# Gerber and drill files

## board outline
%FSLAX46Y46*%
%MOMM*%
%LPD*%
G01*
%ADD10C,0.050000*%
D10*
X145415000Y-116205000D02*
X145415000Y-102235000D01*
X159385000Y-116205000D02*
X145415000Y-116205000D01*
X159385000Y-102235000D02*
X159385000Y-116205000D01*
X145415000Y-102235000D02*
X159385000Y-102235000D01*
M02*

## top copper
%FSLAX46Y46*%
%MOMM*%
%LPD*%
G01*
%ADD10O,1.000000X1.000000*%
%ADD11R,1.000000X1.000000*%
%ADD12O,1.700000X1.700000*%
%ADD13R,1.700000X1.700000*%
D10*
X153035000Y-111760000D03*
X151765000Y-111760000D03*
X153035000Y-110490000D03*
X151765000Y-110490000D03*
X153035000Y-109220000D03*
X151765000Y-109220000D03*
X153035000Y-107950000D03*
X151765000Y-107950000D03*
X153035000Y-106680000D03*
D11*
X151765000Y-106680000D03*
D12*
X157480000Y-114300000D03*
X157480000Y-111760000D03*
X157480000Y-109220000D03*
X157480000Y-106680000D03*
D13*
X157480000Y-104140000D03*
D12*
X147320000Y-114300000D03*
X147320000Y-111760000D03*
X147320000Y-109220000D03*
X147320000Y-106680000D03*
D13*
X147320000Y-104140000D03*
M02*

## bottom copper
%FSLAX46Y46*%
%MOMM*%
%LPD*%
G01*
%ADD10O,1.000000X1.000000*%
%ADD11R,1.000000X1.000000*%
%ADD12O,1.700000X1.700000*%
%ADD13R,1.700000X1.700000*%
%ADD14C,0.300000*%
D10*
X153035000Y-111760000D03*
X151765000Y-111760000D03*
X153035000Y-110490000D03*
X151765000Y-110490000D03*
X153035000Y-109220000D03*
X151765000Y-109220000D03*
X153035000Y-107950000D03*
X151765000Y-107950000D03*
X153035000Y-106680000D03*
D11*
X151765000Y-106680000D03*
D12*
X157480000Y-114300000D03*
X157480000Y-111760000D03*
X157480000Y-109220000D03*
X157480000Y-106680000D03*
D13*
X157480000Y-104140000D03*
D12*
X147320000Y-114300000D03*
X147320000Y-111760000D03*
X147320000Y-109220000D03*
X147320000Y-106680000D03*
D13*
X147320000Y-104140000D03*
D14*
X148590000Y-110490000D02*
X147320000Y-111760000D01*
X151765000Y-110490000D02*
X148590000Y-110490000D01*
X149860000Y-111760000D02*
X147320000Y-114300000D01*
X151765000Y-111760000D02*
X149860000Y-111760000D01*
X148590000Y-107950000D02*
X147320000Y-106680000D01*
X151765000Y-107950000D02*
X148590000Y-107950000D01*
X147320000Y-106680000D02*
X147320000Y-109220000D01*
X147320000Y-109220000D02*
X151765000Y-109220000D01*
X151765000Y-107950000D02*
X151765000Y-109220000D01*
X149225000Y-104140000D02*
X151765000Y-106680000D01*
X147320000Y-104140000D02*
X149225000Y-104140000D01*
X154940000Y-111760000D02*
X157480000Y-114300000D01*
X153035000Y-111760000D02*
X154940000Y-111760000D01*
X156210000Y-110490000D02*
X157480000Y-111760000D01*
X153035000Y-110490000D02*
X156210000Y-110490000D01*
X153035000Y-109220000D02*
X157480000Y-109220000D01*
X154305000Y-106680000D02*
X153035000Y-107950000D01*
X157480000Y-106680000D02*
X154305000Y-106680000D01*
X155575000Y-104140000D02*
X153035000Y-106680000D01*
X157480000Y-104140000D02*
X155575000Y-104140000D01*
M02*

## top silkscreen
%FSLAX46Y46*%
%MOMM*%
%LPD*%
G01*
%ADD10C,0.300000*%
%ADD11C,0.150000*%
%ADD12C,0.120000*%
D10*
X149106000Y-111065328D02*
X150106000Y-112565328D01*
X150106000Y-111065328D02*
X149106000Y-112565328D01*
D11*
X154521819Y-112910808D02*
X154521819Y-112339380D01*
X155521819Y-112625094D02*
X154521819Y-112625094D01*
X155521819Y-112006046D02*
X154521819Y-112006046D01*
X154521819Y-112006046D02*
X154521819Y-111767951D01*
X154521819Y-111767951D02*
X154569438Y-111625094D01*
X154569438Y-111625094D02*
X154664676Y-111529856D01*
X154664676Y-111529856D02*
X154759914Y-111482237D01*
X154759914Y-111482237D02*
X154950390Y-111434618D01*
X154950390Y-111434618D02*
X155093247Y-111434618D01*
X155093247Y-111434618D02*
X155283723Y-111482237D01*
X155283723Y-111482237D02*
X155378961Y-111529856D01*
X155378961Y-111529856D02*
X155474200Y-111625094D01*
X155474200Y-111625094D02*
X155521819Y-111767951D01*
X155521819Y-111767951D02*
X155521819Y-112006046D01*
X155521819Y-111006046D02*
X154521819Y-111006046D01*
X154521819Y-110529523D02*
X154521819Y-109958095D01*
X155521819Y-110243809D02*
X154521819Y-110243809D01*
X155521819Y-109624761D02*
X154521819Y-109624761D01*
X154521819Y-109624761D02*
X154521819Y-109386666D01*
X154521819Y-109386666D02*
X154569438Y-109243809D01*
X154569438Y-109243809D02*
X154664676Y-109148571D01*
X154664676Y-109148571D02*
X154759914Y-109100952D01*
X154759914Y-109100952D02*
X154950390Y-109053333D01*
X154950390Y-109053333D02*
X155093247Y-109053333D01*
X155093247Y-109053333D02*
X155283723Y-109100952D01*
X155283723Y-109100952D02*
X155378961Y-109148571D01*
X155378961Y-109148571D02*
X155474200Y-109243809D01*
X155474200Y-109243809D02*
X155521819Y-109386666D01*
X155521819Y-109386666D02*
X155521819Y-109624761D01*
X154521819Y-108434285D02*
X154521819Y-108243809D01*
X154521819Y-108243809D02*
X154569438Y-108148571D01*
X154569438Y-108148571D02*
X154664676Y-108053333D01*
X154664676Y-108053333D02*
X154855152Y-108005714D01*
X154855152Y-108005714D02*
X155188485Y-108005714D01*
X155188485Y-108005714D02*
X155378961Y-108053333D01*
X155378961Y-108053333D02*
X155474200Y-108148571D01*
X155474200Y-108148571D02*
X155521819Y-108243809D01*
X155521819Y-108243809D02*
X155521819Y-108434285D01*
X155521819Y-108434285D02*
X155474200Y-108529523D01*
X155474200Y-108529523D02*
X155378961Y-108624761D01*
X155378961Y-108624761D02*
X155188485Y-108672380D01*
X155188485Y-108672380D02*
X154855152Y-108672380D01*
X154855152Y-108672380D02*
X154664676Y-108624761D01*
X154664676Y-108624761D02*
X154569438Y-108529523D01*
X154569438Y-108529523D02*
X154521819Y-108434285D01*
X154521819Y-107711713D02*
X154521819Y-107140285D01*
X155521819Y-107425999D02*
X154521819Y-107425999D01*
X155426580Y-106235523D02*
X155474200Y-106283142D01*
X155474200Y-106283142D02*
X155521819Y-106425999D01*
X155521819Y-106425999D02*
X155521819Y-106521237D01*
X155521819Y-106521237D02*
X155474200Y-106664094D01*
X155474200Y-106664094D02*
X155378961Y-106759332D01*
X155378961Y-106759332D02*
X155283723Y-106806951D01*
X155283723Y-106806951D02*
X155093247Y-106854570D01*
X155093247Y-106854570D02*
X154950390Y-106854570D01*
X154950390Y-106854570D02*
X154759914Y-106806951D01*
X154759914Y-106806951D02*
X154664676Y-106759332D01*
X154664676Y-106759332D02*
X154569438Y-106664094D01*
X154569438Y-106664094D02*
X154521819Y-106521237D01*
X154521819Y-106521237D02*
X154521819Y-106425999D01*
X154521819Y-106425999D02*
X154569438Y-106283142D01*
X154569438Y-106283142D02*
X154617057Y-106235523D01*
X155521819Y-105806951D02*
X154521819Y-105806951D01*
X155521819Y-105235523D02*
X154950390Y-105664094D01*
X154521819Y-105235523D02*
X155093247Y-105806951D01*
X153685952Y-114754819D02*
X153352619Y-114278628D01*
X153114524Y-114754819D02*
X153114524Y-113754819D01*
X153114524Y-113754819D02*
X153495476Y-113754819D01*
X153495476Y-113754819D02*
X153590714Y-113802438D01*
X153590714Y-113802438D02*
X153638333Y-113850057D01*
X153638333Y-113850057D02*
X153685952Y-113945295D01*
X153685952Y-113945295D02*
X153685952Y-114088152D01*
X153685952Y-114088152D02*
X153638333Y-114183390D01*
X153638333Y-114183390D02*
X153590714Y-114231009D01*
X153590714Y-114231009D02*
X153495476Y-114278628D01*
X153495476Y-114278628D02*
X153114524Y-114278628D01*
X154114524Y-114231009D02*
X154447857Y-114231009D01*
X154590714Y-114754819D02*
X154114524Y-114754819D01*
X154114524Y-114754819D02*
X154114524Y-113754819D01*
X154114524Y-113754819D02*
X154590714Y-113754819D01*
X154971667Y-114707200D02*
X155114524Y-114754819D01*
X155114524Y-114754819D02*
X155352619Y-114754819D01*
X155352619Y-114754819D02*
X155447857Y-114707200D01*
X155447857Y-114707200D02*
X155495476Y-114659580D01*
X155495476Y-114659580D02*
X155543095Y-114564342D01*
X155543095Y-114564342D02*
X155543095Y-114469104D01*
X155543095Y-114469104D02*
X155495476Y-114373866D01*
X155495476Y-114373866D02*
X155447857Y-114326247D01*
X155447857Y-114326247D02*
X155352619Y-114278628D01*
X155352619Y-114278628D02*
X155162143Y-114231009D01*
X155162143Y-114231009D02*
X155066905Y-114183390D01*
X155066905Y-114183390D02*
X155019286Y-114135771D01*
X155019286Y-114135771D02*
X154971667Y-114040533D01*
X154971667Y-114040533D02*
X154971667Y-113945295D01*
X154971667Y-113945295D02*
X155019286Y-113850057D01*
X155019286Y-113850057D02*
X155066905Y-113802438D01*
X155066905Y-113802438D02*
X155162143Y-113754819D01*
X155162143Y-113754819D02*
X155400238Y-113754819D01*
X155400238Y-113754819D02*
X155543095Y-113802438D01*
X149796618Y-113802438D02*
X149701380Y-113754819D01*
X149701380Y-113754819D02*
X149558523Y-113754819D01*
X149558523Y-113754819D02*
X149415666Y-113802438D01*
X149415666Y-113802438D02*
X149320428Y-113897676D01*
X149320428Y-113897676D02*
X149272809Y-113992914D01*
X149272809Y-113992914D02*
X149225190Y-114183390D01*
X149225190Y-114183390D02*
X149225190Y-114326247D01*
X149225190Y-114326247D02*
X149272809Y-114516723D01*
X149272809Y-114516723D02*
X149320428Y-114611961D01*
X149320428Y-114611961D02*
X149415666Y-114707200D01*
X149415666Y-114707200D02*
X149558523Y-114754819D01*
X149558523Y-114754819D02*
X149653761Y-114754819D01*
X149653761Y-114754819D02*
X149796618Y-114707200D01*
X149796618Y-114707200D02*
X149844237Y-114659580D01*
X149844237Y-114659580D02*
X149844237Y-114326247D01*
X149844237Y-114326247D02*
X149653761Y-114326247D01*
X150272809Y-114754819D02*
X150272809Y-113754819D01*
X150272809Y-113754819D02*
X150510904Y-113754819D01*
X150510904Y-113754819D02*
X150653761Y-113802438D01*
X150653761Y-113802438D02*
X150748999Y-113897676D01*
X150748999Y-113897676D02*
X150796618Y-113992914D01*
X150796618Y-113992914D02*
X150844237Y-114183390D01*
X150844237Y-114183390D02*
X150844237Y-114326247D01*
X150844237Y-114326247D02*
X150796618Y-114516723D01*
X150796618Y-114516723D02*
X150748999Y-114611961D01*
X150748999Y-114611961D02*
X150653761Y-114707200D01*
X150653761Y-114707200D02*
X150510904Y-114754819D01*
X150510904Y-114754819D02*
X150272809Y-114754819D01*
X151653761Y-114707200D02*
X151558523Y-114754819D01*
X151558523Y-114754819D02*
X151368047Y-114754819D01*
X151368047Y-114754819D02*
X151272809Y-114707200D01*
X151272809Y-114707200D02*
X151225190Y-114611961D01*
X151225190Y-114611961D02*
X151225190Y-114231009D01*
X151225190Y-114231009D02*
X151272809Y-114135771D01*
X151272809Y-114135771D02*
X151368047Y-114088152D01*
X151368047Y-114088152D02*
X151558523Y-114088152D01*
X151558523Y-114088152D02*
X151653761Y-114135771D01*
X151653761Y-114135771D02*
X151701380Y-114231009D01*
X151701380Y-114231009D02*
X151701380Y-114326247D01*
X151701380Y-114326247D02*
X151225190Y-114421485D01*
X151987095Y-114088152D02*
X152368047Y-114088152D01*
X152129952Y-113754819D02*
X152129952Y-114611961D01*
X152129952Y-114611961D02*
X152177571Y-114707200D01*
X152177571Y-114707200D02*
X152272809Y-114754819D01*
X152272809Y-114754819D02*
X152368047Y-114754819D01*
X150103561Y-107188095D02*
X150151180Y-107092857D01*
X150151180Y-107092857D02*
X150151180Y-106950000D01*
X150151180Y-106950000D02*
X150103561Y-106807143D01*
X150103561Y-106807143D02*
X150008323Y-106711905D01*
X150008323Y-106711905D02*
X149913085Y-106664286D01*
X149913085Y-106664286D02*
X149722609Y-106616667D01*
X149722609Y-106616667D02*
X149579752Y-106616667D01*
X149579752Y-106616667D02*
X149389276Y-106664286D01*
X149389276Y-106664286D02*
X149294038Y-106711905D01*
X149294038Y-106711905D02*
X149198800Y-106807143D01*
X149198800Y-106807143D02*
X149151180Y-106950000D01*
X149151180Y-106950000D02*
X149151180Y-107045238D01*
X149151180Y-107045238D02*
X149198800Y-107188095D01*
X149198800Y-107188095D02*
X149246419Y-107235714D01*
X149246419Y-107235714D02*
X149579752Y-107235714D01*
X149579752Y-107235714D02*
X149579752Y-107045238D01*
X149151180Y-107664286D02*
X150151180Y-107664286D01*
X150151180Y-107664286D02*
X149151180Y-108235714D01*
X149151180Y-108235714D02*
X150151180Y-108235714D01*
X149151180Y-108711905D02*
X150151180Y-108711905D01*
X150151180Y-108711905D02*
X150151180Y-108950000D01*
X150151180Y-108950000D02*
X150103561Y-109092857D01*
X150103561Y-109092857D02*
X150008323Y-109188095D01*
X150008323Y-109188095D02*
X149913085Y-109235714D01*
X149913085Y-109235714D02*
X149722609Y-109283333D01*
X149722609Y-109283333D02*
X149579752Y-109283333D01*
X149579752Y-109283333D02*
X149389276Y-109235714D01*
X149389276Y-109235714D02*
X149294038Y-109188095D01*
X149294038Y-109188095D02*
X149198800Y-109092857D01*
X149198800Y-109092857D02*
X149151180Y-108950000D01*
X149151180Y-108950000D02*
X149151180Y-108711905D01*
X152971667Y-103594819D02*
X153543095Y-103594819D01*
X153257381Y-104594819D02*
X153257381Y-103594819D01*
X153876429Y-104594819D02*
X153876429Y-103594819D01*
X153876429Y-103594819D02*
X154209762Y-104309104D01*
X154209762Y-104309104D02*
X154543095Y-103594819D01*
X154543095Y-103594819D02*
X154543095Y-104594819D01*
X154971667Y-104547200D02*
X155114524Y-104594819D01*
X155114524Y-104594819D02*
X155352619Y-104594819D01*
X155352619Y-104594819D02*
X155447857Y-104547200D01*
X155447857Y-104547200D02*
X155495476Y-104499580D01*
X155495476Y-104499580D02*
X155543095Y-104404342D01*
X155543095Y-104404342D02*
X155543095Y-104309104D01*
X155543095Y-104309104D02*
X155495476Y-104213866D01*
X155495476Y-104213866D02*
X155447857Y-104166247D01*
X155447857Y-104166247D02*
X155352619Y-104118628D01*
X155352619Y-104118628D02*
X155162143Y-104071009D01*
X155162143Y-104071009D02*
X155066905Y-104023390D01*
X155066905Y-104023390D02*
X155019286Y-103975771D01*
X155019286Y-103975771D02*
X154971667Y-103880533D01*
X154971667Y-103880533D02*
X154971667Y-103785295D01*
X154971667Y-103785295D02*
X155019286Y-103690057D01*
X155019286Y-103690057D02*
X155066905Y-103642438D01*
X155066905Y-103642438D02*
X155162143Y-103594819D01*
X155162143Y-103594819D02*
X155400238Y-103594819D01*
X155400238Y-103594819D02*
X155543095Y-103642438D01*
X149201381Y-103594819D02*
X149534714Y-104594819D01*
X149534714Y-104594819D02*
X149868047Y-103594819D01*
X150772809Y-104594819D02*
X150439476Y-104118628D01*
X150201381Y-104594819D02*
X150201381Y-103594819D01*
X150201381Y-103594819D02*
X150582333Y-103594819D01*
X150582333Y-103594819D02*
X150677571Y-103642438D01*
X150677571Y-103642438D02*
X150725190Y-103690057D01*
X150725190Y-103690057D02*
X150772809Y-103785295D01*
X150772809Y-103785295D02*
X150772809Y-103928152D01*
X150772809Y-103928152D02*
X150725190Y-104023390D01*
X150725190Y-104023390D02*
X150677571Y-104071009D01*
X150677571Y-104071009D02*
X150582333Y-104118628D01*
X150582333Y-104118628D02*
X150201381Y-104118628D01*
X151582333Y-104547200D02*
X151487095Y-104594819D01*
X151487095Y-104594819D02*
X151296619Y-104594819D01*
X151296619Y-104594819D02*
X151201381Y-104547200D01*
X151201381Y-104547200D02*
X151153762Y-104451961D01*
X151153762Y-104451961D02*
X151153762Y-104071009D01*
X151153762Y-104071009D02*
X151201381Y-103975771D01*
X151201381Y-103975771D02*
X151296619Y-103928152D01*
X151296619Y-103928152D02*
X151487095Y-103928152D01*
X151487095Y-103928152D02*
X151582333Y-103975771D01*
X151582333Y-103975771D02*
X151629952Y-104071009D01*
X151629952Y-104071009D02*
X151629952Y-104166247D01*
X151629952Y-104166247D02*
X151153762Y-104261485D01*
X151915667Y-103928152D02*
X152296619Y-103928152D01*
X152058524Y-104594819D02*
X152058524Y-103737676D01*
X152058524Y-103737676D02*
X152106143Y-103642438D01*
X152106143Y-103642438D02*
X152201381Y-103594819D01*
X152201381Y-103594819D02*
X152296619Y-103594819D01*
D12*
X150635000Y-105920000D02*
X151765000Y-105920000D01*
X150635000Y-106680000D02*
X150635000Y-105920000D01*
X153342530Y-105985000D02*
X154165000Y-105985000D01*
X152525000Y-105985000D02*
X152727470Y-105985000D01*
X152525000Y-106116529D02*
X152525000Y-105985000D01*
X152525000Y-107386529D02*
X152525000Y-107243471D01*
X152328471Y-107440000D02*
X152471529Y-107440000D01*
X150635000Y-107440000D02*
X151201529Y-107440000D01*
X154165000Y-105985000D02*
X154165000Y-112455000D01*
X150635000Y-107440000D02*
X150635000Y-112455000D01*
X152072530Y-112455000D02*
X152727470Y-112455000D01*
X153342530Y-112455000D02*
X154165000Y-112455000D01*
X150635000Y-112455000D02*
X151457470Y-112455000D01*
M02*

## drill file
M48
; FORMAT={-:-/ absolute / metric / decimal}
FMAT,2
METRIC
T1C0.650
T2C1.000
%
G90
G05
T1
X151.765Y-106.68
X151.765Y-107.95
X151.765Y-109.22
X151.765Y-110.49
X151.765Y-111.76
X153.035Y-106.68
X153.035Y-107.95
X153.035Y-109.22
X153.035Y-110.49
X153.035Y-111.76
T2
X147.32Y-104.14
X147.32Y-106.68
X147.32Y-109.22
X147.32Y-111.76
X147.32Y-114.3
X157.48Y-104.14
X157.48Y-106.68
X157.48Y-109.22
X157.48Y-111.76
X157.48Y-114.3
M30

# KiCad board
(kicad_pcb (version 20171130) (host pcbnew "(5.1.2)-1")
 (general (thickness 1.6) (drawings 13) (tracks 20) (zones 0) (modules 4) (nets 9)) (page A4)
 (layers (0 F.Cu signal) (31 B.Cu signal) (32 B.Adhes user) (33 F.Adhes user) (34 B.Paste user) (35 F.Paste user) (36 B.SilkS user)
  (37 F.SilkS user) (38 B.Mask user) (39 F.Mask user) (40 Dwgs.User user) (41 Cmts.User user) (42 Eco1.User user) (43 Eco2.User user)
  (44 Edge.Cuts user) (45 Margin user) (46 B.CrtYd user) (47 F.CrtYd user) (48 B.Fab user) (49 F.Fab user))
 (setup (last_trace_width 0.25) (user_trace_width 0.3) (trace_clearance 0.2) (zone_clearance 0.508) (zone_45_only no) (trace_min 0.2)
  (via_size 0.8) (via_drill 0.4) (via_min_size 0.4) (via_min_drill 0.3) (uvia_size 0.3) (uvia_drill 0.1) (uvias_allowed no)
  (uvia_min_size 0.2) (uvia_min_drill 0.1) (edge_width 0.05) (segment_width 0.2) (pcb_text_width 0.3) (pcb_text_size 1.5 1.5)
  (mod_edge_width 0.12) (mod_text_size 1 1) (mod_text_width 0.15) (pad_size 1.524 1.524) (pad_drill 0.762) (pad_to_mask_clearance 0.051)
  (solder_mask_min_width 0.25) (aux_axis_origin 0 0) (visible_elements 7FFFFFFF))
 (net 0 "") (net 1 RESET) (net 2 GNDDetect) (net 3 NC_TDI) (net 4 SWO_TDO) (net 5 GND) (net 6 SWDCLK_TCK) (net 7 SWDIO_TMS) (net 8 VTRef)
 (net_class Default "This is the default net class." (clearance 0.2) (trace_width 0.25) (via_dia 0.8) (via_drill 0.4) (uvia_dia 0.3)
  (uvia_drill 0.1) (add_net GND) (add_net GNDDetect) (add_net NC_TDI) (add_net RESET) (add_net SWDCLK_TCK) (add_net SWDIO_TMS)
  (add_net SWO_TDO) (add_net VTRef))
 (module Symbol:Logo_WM (layer B.Cu) (at 152.527 114.427)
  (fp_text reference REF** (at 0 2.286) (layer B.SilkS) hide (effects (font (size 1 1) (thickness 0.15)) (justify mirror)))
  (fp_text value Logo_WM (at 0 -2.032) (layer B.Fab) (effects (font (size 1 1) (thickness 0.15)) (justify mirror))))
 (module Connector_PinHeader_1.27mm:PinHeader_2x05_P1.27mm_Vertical (layer F.Cu) (at 151.765 106.68)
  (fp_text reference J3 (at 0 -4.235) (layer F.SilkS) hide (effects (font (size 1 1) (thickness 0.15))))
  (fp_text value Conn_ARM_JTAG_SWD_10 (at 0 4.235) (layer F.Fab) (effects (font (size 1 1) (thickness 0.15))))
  (fp_line (start -1.13 -0.76) (end 0 -0.76) (layer F.SilkS) (width 0.12))
  (fp_line (start -1.13 0) (end -1.13 -0.76) (layer F.SilkS) (width 0.12))
  (fp_line (start 1.57753 -0.695) (end 2.4 -0.695) (layer F.SilkS) (width 0.12))
  (fp_line (start 0.76 -0.695) (end 0.96247 -0.695) (layer F.SilkS) (width 0.12))
  (fp_line (start 0.76 -0.563471) (end 0.76 -0.695) (layer F.SilkS) (width 0.12))
  (fp_line (start 0.76 0.706529) (end 0.76 0.563471) (layer F.SilkS) (width 0.12))
  (fp_line (start 0.563471 0.76) (end 0.706529 0.76) (layer F.SilkS) (width 0.12))
  (fp_line (start -1.13 0.76) (end -0.563471 0.76) (layer F.SilkS) (width 0.12))
  (fp_line (start 2.4 -0.695) (end 2.4 5.775) (layer F.SilkS) (width 0.12))
  (fp_line (start -1.13 0.76) (end -1.13 5.775) (layer F.SilkS) (width 0.12))
  (fp_line (start 0.30753 5.775) (end 0.96247 5.775) (layer F.SilkS) (width 0.12))
  (fp_line (start 1.57753 5.775) (end 2.4 5.775) (layer F.SilkS) (width 0.12))
  (fp_line (start -1.13 5.775) (end -0.30753 5.775) (layer F.SilkS) (width 0.12))
  (pad 10 thru_hole oval (at 1.27 5.08) (size 1 1) (drill 0.65) (layers *.Cu *.Mask) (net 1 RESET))
  (pad 9 thru_hole oval (at 0 5.08) (size 1 1) (drill 0.65) (layers *.Cu *.Mask) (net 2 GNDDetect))
  (pad 8 thru_hole oval (at 1.27 3.81) (size 1 1) (drill 0.65) (layers *.Cu *.Mask) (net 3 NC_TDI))
  (pad 7 thru_hole oval (at 0 3.81) (size 1 1) (drill 0.65) (layers *.Cu *.Mask))
  (pad 6 thru_hole oval (at 1.27 2.54) (size 1 1) (drill 0.65) (layers *.Cu *.Mask) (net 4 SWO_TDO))
  (pad 5 thru_hole oval (at 0 2.54) (size 1 1) (drill 0.65) (layers *.Cu *.Mask) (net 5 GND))
  (pad 4 thru_hole oval (at 1.27 1.27) (size 1 1) (drill 0.65) (layers *.Cu *.Mask) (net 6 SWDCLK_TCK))
  (pad 3 thru_hole oval (at 0 1.27) (size 1 1) (drill 0.65) (layers *.Cu *.Mask) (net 5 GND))
  (pad 2 thru_hole oval (at 1.27 0) (size 1 1) (drill 0.65) (layers *.Cu *.Mask) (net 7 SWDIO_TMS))
  (pad 1 thru_hole rect (at 0 0) (size 1 1) (drill 0.65) (layers *.Cu *.Mask) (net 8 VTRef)))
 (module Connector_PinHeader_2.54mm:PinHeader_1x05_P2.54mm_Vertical (layer B.Cu) (at 157.48 104.14 180)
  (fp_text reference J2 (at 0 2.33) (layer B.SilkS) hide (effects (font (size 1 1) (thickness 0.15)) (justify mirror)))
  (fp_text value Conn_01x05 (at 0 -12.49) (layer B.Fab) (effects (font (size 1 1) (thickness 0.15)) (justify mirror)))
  (pad 5 thru_hole oval (at 0 -10.16 180) (size 1.7 1.7) (drill 1) (layers *.Cu *.Mask) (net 1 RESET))
  (pad 4 thru_hole oval (at 0 -7.62 180) (size 1.7 1.7) (drill 1) (layers *.Cu *.Mask) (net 3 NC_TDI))
  (pad 3 thru_hole oval (at 0 -5.08 180) (size 1.7 1.7) (drill 1) (layers *.Cu *.Mask) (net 4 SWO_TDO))
  (pad 2 thru_hole oval (at 0 -2.54 180) (size 1.7 1.7) (drill 1) (layers *.Cu *.Mask) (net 6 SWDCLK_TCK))
  (pad 1 thru_hole rect (at 0 0 180) (size 1.7 1.7) (drill 1) (layers *.Cu *.Mask) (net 7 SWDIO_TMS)))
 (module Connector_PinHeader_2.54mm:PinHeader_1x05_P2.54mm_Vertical (layer B.Cu) (at 147.32 104.14 180)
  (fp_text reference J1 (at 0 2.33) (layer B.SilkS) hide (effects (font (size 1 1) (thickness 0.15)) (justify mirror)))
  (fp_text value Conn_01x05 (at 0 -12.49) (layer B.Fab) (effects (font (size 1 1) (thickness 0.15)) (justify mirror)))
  (pad 5 thru_hole oval (at 0 -10.16 180) (size 1.7 1.7) (drill 1) (layers *.Cu *.Mask) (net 2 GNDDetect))
  (pad 4 thru_hole oval (at 0 -7.62 180) (size 1.7 1.7) (drill 1) (layers *.Cu *.Mask))
  (pad 3 thru_hole oval (at 0 -5.08 180) (size 1.7 1.7) (drill 1) (layers *.Cu *.Mask) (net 5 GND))
  (pad 2 thru_hole oval (at 0 -2.54 180) (size 1.7 1.7) (drill 1) (layers *.Cu *.Mask) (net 5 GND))
  (pad 1 thru_hole rect (at 0 0 180) (size 1.7 1.7) (drill 1) (layers *.Cu *.Mask) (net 8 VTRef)))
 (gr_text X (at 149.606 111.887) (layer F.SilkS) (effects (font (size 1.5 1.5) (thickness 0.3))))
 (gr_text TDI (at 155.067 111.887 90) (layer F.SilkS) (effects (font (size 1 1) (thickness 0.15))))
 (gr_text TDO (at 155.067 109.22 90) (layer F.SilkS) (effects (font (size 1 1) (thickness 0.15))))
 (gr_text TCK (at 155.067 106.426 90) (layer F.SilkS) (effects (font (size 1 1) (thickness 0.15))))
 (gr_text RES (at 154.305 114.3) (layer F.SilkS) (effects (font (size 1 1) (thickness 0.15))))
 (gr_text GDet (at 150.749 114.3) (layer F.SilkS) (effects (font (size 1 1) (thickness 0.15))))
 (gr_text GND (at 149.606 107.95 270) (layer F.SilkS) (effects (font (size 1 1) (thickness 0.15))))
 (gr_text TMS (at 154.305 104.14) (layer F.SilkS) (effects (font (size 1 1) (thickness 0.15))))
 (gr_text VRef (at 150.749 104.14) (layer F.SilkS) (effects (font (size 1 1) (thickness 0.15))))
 (gr_line (start 145.415 116.205) (end 145.415 102.235) (layer Edge.Cuts) (width 0.05))
 (gr_line (start 159.385 116.205) (end 145.415 116.205) (layer Edge.Cuts) (width 0.05))
 (gr_line (start 159.385 102.235) (end 159.385 116.205) (layer Edge.Cuts) (width 0.05))
 (gr_line (start 145.415 102.235) (end 159.385 102.235) (layer Edge.Cuts) (width 0.05))
 (segment (start 148.59 110.49) (end 147.32 111.76) (width 0.3) (layer B.Cu) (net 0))
 (segment (start 151.765 110.49) (end 148.59 110.49) (width 0.3) (layer B.Cu) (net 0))
 (segment (start 149.86 111.76) (end 147.32 114.3) (width 0.3) (layer B.Cu) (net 2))
 (segment (start 151.765 111.76) (end 149.86 111.76) (width 0.3) (layer B.Cu) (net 2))
 (segment (start 148.59 107.95) (end 147.32 106.68) (width 0.3) (layer B.Cu) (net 5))
 (segment (start 151.765 107.95) (end 148.59 107.95) (width 0.3) (layer B.Cu) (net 5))
 (segment (start 147.32 106.68) (end 147.32 109.22) (width 0.3) (layer B.Cu) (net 5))
 (segment (start 147.32 109.22) (end 151.765 109.22) (width 0.3) (layer B.Cu) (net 5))
 (segment (start 151.765 107.95) (end 151.765 109.22) (width 0.3) (layer B.Cu) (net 5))
 (segment (start 149.225 104.14) (end 151.765 106.68) (width 0.3) (layer B.Cu) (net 8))
 (segment (start 147.32 104.14) (end 149.225 104.14) (width 0.3) (layer B.Cu) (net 8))
 (segment (start 154.94 111.76) (end 157.48 114.3) (width 0.3) (layer B.Cu) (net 1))
 (segment (start 153.035 111.76) (end 154.94 111.76) (width 0.3) (layer B.Cu) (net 1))
 (segment (start 156.21 110.49) (end 157.48 111.76) (width 0.3) (layer B.Cu) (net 3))
 (segment (start 153.035 110.49) (end 156.21 110.49) (width 0.3) (layer B.Cu) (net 3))
 (segment (start 153.035 109.22) (end 157.48 109.22) (width 0.3) (layer B.Cu) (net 4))
 (segment (start 154.305 106.68) (end 153.035 107.95) (width 0.3) (layer B.Cu) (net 6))
 (segment (start 157.48 106.68) (end 154.305 106.68) (width 0.3) (layer B.Cu) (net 6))
 (segment (start 155.575 104.14) (end 153.035 106.68) (width 0.3) (layer B.Cu) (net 7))
 (segment (start 157.48 104.14) (end 155.575 104.14) (width 0.3) (layer B.Cu) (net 7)))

